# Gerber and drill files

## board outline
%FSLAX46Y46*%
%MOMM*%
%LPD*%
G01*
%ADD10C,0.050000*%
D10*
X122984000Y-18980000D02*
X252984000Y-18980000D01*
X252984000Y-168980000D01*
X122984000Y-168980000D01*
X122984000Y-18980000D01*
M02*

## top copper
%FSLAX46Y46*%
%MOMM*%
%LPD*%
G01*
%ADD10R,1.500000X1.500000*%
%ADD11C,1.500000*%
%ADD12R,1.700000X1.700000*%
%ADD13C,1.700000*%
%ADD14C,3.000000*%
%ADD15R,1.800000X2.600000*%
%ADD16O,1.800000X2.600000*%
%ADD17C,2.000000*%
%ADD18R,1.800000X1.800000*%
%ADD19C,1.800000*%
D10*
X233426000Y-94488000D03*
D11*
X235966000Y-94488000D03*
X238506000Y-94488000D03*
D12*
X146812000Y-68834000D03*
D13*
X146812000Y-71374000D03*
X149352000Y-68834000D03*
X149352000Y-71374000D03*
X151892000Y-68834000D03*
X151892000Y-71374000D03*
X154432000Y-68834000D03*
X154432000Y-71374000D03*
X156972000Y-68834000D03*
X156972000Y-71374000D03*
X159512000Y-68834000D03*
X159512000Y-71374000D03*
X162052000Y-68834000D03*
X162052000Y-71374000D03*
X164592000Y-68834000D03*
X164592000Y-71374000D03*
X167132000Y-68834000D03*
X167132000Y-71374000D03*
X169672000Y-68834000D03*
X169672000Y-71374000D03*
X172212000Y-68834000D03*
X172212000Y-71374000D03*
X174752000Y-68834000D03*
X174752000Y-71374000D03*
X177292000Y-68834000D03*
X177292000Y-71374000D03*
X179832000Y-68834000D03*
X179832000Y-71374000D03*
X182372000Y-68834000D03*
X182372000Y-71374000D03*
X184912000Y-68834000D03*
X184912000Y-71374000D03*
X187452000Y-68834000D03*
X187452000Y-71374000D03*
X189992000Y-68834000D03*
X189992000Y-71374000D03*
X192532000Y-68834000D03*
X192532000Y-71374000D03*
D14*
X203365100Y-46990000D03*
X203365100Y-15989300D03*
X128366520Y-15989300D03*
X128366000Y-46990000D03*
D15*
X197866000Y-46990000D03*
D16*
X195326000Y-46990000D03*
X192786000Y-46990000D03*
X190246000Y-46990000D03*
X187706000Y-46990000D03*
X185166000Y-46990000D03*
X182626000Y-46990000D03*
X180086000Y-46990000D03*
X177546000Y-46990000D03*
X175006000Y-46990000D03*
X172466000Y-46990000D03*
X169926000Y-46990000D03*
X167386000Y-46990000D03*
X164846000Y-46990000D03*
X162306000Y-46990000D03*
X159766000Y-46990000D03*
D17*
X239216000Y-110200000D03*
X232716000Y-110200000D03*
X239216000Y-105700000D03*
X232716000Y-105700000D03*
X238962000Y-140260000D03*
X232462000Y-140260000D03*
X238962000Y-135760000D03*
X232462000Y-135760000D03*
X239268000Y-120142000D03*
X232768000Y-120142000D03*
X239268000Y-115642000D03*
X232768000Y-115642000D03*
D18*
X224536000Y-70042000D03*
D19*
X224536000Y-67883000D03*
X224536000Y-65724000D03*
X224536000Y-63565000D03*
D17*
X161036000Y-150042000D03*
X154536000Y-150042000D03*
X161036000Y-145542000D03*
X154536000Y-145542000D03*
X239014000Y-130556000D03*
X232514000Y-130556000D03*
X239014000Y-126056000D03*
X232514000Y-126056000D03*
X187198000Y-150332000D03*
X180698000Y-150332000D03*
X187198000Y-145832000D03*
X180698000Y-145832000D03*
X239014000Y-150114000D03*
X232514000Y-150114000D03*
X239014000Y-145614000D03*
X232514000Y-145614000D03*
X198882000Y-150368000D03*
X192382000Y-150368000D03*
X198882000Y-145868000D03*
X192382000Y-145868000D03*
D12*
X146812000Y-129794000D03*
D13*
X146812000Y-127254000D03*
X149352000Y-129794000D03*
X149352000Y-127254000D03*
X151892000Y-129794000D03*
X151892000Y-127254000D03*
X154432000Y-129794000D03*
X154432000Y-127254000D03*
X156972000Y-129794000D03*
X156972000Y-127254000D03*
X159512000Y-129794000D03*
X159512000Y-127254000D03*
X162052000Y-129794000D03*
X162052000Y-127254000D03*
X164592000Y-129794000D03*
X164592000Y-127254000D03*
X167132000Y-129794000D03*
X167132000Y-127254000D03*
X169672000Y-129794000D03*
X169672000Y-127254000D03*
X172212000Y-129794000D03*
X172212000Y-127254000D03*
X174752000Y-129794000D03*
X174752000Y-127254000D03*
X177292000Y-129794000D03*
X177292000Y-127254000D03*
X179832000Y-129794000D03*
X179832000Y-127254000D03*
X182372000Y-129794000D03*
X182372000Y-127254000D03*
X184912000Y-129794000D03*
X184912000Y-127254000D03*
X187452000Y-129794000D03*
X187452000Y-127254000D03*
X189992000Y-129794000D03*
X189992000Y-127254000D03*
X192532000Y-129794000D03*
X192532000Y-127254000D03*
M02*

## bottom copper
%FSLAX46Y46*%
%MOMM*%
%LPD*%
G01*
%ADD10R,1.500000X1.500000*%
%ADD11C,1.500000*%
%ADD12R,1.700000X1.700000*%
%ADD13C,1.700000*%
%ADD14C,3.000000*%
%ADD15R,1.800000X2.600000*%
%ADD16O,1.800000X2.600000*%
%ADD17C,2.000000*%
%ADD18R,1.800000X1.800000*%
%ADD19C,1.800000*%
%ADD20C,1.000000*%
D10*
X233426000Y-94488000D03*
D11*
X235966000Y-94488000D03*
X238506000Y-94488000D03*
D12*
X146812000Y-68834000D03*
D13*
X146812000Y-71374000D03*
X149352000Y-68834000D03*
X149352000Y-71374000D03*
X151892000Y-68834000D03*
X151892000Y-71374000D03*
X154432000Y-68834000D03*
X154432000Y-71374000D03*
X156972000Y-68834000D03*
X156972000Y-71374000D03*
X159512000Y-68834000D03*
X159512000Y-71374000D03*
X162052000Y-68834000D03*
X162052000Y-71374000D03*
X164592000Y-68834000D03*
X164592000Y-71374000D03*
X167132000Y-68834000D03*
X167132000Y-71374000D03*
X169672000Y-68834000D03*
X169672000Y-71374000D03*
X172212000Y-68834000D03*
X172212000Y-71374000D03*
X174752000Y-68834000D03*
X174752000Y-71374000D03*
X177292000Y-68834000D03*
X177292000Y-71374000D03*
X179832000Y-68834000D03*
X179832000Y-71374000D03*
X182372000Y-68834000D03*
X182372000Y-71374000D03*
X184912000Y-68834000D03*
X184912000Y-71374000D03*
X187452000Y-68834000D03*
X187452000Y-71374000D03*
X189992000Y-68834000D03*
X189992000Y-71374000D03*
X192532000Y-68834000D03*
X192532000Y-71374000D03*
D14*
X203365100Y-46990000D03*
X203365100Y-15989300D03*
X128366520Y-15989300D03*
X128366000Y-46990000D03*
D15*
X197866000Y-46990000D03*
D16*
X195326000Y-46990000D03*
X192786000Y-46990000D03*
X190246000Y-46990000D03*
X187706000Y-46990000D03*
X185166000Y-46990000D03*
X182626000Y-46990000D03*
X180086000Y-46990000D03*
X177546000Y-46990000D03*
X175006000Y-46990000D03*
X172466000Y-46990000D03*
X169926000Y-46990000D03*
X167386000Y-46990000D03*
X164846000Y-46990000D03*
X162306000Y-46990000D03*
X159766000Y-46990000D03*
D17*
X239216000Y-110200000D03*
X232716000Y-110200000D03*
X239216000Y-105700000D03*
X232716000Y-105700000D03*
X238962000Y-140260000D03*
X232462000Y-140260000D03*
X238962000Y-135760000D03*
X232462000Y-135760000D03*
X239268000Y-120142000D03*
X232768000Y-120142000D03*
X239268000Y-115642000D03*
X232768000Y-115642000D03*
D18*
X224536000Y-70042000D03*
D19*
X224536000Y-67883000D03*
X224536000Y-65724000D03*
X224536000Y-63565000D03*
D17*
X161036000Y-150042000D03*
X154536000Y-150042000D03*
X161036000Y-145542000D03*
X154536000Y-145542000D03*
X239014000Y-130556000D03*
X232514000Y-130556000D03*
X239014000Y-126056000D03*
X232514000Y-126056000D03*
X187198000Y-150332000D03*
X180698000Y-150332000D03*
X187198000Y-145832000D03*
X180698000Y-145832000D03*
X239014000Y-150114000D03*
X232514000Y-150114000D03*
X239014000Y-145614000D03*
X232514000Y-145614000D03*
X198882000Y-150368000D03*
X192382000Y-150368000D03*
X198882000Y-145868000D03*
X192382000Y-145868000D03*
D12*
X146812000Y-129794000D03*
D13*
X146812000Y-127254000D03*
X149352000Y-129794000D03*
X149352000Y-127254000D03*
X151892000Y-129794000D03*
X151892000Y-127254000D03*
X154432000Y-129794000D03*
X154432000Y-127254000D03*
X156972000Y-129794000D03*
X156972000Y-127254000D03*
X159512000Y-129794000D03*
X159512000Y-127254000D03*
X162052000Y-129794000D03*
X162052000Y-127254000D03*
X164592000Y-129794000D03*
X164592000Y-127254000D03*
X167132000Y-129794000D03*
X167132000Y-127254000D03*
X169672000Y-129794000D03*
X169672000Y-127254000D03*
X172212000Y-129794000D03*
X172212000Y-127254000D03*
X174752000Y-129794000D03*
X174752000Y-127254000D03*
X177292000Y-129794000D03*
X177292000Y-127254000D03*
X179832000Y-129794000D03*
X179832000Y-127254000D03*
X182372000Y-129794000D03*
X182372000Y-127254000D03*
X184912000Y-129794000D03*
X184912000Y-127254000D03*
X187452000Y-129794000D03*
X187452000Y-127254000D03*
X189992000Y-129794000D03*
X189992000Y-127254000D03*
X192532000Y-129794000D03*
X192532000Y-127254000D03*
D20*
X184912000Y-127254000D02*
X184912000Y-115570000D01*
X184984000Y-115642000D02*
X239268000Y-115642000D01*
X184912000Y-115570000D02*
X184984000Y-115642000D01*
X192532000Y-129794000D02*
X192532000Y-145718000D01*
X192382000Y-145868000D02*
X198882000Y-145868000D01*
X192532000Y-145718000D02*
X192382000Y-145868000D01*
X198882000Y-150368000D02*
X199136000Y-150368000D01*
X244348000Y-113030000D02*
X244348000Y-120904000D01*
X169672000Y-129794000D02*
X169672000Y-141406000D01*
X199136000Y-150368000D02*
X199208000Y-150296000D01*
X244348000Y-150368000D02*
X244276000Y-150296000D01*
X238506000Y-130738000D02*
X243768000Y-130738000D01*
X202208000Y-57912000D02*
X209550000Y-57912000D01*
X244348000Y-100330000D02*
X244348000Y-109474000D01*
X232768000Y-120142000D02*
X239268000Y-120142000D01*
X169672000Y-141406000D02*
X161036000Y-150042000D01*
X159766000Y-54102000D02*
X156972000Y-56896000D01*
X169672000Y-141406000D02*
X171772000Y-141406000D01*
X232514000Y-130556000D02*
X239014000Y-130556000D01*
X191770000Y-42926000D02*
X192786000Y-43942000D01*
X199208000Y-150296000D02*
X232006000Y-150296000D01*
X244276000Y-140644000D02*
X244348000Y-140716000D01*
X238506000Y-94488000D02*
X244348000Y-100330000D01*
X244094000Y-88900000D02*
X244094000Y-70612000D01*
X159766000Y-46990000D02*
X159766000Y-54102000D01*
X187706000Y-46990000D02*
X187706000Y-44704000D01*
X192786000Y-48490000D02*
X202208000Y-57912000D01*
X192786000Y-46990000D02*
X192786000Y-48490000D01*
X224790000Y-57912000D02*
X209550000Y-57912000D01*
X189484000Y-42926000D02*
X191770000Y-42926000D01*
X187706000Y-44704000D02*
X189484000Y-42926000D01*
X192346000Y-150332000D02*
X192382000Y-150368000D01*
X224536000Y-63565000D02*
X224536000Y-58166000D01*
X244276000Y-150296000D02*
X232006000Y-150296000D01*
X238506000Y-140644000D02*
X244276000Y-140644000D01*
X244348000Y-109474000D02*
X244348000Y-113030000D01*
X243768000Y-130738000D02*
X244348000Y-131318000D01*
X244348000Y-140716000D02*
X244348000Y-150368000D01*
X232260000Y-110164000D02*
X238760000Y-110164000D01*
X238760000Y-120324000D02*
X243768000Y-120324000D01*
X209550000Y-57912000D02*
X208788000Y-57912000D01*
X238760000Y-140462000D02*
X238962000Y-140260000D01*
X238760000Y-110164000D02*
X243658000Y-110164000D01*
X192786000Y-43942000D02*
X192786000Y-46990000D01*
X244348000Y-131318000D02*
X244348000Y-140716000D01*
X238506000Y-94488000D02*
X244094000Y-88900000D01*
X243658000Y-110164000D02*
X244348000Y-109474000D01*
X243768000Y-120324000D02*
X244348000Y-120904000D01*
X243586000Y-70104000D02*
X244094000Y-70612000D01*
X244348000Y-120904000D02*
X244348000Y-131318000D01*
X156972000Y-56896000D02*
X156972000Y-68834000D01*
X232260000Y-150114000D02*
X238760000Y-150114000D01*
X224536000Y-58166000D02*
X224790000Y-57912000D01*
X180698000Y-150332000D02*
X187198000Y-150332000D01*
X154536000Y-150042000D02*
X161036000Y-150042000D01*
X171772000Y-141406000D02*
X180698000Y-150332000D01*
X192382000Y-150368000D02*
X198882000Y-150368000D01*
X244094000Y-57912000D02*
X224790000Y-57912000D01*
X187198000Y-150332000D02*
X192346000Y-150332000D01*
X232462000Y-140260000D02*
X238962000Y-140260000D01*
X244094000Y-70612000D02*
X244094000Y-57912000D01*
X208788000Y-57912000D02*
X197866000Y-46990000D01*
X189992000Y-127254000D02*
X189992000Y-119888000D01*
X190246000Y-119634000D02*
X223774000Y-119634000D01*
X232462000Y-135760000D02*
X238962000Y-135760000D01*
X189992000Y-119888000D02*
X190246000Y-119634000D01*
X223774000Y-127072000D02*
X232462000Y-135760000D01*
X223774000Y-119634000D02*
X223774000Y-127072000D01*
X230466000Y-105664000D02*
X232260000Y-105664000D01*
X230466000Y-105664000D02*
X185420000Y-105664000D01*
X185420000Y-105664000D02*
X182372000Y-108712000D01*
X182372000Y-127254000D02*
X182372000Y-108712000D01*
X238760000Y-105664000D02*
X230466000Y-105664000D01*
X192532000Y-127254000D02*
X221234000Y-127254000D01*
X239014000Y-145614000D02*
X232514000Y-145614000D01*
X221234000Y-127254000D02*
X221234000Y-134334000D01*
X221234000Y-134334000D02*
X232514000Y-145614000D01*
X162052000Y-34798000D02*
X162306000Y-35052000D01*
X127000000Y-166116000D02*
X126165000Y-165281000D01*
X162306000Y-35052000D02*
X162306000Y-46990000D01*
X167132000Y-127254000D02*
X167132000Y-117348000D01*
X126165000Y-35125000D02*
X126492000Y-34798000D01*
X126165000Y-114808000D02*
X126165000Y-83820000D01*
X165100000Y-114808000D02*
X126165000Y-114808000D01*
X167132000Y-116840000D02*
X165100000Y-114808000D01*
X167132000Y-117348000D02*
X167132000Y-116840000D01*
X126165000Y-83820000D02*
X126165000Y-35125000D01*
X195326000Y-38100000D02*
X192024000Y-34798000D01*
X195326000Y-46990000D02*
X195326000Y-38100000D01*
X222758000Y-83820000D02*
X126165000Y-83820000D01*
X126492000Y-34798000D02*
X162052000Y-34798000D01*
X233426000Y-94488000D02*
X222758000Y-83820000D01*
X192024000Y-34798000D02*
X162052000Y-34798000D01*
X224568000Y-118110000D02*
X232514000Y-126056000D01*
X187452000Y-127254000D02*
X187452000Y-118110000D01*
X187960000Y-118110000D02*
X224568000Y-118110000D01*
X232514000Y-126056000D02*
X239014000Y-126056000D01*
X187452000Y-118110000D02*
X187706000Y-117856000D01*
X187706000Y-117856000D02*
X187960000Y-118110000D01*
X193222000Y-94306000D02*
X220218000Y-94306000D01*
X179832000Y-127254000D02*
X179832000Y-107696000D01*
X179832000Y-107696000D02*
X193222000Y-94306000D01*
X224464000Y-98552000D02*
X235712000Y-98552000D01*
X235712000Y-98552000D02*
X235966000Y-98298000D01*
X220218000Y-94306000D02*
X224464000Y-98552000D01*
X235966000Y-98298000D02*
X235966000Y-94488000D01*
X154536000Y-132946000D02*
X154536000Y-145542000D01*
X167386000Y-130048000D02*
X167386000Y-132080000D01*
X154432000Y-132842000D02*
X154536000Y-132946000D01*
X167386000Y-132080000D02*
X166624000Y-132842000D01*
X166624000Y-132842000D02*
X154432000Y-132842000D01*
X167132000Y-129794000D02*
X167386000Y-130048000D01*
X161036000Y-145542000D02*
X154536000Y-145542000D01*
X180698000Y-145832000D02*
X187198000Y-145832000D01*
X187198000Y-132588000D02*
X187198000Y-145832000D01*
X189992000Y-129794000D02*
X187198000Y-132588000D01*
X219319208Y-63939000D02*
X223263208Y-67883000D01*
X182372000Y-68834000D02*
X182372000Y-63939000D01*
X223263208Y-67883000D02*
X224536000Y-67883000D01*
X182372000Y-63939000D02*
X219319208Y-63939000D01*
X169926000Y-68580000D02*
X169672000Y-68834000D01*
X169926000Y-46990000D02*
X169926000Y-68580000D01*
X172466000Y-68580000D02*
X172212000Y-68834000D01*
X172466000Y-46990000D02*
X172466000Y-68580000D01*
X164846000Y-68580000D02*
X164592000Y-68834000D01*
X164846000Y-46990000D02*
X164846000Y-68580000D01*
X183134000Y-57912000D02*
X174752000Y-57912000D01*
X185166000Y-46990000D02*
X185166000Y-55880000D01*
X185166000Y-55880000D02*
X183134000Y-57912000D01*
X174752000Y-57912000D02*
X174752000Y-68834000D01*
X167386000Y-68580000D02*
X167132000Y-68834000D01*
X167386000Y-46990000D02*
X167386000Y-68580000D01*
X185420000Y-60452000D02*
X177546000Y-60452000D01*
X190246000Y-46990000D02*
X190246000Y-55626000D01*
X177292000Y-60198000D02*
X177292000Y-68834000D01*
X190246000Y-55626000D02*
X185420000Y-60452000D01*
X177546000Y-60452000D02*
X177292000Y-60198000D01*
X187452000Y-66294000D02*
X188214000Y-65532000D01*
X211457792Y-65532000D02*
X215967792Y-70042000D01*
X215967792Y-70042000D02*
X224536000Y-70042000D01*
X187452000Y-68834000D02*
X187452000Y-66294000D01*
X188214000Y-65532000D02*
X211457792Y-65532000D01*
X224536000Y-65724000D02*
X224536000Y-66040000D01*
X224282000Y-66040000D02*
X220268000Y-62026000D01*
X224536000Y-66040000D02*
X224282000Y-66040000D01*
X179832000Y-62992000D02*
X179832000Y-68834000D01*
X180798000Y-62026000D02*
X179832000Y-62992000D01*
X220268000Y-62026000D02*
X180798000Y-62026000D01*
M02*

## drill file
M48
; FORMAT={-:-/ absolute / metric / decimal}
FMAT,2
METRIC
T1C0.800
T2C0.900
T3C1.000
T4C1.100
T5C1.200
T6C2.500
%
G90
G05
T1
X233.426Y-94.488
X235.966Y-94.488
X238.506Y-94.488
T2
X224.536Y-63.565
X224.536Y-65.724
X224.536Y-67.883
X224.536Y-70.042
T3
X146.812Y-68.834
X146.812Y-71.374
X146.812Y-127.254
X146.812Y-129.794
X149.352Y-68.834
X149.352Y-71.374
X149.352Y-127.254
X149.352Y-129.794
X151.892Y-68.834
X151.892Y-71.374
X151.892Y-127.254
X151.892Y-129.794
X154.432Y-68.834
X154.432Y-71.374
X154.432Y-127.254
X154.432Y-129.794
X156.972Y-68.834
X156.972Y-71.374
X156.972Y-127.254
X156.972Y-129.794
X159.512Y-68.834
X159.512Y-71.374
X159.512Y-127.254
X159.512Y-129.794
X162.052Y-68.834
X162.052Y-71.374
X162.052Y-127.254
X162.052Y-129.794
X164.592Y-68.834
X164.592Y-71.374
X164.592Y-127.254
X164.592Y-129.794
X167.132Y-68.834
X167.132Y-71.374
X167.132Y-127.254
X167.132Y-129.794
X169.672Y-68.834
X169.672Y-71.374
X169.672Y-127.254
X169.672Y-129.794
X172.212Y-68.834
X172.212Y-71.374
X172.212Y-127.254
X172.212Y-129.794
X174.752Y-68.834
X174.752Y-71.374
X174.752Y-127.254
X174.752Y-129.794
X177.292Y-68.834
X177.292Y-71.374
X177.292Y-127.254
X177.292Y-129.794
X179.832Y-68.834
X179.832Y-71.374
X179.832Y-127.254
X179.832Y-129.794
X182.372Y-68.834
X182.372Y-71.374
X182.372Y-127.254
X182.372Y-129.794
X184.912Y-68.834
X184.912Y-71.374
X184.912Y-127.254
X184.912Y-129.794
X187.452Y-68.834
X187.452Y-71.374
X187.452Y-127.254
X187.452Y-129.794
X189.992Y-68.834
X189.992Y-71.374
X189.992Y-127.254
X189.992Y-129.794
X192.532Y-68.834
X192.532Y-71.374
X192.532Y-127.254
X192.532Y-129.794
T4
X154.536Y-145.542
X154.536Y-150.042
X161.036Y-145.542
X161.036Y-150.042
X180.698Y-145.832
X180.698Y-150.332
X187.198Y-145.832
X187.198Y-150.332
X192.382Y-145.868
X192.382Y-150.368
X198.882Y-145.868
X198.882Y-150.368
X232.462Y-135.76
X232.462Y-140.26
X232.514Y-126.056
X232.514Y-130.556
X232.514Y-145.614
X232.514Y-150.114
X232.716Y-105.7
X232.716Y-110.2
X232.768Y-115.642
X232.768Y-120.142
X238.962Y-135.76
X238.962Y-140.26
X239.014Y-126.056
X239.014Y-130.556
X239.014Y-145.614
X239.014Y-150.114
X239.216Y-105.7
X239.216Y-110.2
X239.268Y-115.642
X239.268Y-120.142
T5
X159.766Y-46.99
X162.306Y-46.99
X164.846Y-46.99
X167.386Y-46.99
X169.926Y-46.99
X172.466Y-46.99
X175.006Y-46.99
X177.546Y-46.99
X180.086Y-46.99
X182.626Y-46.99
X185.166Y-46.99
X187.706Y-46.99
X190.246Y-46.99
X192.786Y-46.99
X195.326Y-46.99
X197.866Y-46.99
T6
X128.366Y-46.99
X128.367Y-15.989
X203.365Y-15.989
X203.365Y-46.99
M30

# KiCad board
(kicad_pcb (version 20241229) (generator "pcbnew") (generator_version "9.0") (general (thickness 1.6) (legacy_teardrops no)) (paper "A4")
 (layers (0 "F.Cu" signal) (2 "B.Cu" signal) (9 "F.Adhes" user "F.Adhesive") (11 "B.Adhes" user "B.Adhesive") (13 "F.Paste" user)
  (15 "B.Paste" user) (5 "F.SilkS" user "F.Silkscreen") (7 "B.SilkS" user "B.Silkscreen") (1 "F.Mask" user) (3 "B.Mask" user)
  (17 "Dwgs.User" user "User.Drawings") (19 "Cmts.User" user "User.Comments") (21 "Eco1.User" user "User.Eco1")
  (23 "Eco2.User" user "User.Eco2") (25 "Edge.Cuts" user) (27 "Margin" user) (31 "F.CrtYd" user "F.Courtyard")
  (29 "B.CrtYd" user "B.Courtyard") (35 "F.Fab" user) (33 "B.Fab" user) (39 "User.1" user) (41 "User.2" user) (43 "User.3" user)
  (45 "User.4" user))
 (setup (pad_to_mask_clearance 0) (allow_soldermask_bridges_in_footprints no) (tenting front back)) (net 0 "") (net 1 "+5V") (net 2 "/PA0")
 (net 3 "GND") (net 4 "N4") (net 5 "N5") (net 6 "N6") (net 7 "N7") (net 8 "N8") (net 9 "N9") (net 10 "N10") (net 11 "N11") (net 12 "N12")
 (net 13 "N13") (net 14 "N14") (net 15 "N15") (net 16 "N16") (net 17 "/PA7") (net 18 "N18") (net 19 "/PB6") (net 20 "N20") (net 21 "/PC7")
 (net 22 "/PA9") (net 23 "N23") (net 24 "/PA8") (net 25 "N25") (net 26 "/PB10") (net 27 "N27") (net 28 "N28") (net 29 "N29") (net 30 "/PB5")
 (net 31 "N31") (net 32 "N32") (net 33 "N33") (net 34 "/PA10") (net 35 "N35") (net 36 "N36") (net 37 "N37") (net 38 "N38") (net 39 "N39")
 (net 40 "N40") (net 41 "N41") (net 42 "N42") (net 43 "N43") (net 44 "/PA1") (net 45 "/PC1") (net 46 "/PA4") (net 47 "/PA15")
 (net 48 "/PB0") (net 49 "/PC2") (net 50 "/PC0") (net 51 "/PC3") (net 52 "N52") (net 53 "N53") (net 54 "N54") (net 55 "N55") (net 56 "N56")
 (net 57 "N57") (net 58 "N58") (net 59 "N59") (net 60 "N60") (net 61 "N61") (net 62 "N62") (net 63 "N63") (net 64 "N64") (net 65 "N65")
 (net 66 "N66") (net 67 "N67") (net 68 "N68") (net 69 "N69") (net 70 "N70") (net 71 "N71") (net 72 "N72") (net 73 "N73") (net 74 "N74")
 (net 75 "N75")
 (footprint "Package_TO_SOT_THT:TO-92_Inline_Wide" (layer "F.Cu") (at 233.426 94.488)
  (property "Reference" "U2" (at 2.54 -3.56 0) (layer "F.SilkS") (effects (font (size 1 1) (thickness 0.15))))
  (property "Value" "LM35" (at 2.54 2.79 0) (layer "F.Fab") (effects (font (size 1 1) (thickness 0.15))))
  (pad "1" thru_hole rect (at 0 0) (size 1.5 1.5) (drill 0.8) (layers "*.Cu" "*.Mask") (remove_unused_layers no) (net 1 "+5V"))
  (pad "2" thru_hole circle (at 2.54 0) (size 1.5 1.5) (drill 0.8) (layers "*.Cu" "*.Mask") (remove_unused_layers no) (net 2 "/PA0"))
  (pad "3" thru_hole circle (at 5.08 0) (size 1.5 1.5) (drill 0.8) (layers "*.Cu" "*.Mask") (remove_unused_layers no) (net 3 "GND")))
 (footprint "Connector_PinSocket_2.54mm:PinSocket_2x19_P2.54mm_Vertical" (layer "F.Cu") (at 146.812 68.834 90)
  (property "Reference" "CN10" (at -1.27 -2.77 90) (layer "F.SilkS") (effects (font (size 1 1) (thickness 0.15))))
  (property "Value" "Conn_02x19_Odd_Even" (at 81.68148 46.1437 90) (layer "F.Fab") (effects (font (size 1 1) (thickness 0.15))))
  (pad "1" thru_hole rect (at 0 0 90) (size 1.7 1.7) (drill 1) (layers "*.Cu" "*.Mask") (remove_unused_layers no) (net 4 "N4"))
  (pad "2" thru_hole circle (at -2.54 0 90) (size 1.7 1.7) (drill 1) (layers "*.Cu" "*.Mask") (remove_unused_layers no) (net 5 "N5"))
  (pad "3" thru_hole circle (at 0 2.54 90) (size 1.7 1.7) (drill 1) (layers "*.Cu" "*.Mask") (remove_unused_layers no) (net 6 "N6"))
  (pad "4" thru_hole circle (at -2.54 2.54 90) (size 1.7 1.7) (drill 1) (layers "*.Cu" "*.Mask") (remove_unused_layers no) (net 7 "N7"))
  (pad "5" thru_hole circle (at 0 5.08 90) (size 1.7 1.7) (drill 1) (layers "*.Cu" "*.Mask") (remove_unused_layers no) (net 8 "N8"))
  (pad "6" thru_hole circle (at -2.54 5.08 90) (size 1.7 1.7) (drill 1) (layers "*.Cu" "*.Mask") (remove_unused_layers no) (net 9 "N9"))
  (pad "7" thru_hole circle (at 0 7.62 90) (size 1.7 1.7) (drill 1) (layers "*.Cu" "*.Mask") (remove_unused_layers no) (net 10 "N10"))
  (pad "8" thru_hole circle (at -2.54 7.62 90) (size 1.7 1.7) (drill 1) (layers "*.Cu" "*.Mask") (remove_unused_layers no) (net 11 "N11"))
  (pad "9" thru_hole circle (at 0 10.16 90) (size 1.7 1.7) (drill 1) (layers "*.Cu" "*.Mask") (remove_unused_layers no) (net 3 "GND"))
  (pad "10" thru_hole circle (at -2.54 10.16 90) (size 1.7 1.7) (drill 1) (layers "*.Cu" "*.Mask") (remove_unused_layers no) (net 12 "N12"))
  (pad "11" thru_hole circle (at 0 12.7 90) (size 1.7 1.7) (drill 1) (layers "*.Cu" "*.Mask") (remove_unused_layers no) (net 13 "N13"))
  (pad "12" thru_hole circle (at -2.54 12.7 90) (size 1.7 1.7) (drill 1) (layers "*.Cu" "*.Mask") (remove_unused_layers no) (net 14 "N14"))
  (pad "13" thru_hole circle (at 0 15.24 90) (size 1.7 1.7) (drill 1) (layers "*.Cu" "*.Mask") (remove_unused_layers no) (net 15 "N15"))
  (pad "14" thru_hole circle (at -2.54 15.24 90) (size 1.7 1.7) (drill 1) (layers "*.Cu" "*.Mask") (remove_unused_layers no) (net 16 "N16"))
  (pad "15" thru_hole circle (at 0 17.78 90) (size 1.7 1.7) (drill 1) (layers "*.Cu" "*.Mask") (remove_unused_layers no) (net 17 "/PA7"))
  (pad "16" thru_hole circle (at -2.54 17.78 90) (size 1.7 1.7) (drill 1) (layers "*.Cu" "*.Mask") (remove_unused_layers no) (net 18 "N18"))
  (pad "17" thru_hole circle (at 0 20.32 90) (size 1.7 1.7) (drill 1) (layers "*.Cu" "*.Mask") (remove_unused_layers no) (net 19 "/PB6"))
  (pad "18" thru_hole circle (at -2.54 20.32 90) (size 1.7 1.7) (drill 1) (layers "*.Cu" "*.Mask") (remove_unused_layers no) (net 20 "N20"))
  (pad "19" thru_hole circle (at 0 22.86 90) (size 1.7 1.7) (drill 1) (layers "*.Cu" "*.Mask") (remove_unused_layers no) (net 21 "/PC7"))
  (pad "20" thru_hole circle (at -2.54 22.86 90) (size 1.7 1.7) (drill 1) (layers "*.Cu" "*.Mask") (remove_unused_layers no) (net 3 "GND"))
  (pad "21" thru_hole circle (at 0 25.4 90) (size 1.7 1.7) (drill 1) (layers "*.Cu" "*.Mask") (remove_unused_layers no) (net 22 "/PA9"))
  (pad "22" thru_hole circle (at -2.54 25.4 90) (size 1.7 1.7) (drill 1) (layers "*.Cu" "*.Mask") (remove_unused_layers no) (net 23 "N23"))
  (pad "23" thru_hole circle (at 0 27.94 90) (size 1.7 1.7) (drill 1) (layers "*.Cu" "*.Mask") (remove_unused_layers no) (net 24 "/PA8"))
  (pad "24" thru_hole circle (at -2.54 27.94 90) (size 1.7 1.7) (drill 1) (layers "*.Cu" "*.Mask") (remove_unused_layers no) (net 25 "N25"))
  (pad "25" thru_hole circle (at 0 30.48 90) (size 1.7 1.7) (drill 1) (layers "*.Cu" "*.Mask") (remove_unused_layers no) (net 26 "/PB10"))
  (pad "26" thru_hole circle (at -2.54 30.48 90) (size 1.7 1.7) (drill 1) (layers "*.Cu" "*.Mask") (remove_unused_layers no) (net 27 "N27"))
  (pad "27" thru_hole circle (at 0 33.02 90) (size 1.7 1.7) (drill 1) (layers "*.Cu" "*.Mask") (remove_unused_layers no) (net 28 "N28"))
  (pad "28" thru_hole circle (at -2.54 33.02 90) (size 1.7 1.7) (drill 1) (layers "*.Cu" "*.Mask") (remove_unused_layers no) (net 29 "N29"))
  (pad "29" thru_hole circle (at 0 35.56 90) (size 1.7 1.7) (drill 1) (layers "*.Cu" "*.Mask") (remove_unused_layers no) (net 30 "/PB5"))
  (pad "30" thru_hole circle (at -2.54 35.56 90) (size 1.7 1.7) (drill 1) (layers "*.Cu" "*.Mask") (remove_unused_layers no) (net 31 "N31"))
  (pad "31" thru_hole circle (at 0 38.1 90) (size 1.7 1.7) (drill 1) (layers "*.Cu" "*.Mask") (remove_unused_layers no) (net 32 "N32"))
  (pad "32" thru_hole circle (at -2.54 38.1 90) (size 1.7 1.7) (drill 1) (layers "*.Cu" "*.Mask") (remove_unused_layers no) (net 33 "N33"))
  (pad "33" thru_hole circle (at 0 40.64 90) (size 1.7 1.7) (drill 1) (layers "*.Cu" "*.Mask") (remove_unused_layers no) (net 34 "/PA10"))
  (pad "34" thru_hole circle (at -2.54 40.64 90) (size 1.7 1.7) (drill 1) (layers "*.Cu" "*.Mask") (remove_unused_layers no) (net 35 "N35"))
  (pad "35" thru_hole circle (at 0 43.18 90) (size 1.7 1.7) (drill 1) (layers "*.Cu" "*.Mask") (remove_unused_layers no) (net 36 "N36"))
  (pad "36" thru_hole circle (at -2.54 43.18 90) (size 1.7 1.7) (drill 1) (layers "*.Cu" "*.Mask") (remove_unused_layers no) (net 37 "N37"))
  (pad "37" thru_hole circle (at 0 45.72 90) (size 1.7 1.7) (drill 1) (layers "*.Cu" "*.Mask") (remove_unused_layers no) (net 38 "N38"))
  (pad "38" thru_hole circle (at -2.54 45.72 90) (size 1.7 1.7) (drill 1) (layers "*.Cu" "*.Mask") (remove_unused_layers no) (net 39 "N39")))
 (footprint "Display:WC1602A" (layer "F.Cu") (at 197.866 46.99 180)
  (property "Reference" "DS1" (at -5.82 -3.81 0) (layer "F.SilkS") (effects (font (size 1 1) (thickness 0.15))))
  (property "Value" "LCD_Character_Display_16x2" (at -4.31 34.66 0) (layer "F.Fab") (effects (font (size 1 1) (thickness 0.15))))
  (pad "" thru_hole circle (at -5.4991 0 180) (size 3 3) (drill 2.5) (layers "*.Cu" "*.Mask") (remove_unused_layers no))
  (pad "" thru_hole circle (at -5.4991 31.0007 180) (size 3 3) (drill 2.5) (layers "*.Cu" "*.Mask") (remove_unused_layers no))
  (pad "" thru_hole circle (at 69.49948 31.0007 180) (size 3 3) (drill 2.5) (layers "*.Cu" "*.Mask") (remove_unused_layers no))
  (pad "" thru_hole circle (at 69.5 0 180) (size 3 3) (drill 2.5) (layers "*.Cu" "*.Mask") (remove_unused_layers no))
  (pad "1" thru_hole rect (at 0 0 180) (size 1.8 2.6) (drill 1.2) (layers "*.Cu" "*.Mask") (remove_unused_layers no) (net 3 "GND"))
  (pad "2" thru_hole oval (at 2.54 0 180) (size 1.8 2.6) (drill 1.2) (layers "*.Cu" "*.Mask") (remove_unused_layers no) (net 1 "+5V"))
  (pad "3" thru_hole oval (at 5.08 0 180) (size 1.8 2.6) (drill 1.2) (layers "*.Cu" "*.Mask") (remove_unused_layers no) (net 3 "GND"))
  (pad "4" thru_hole oval (at 7.62 0 180) (size 1.8 2.6) (drill 1.2) (layers "*.Cu" "*.Mask") (remove_unused_layers no) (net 26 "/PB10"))
  (pad "5" thru_hole oval (at 10.16 0 180) (size 1.8 2.6) (drill 1.2) (layers "*.Cu" "*.Mask") (remove_unused_layers no) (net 3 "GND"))
  (pad "6" thru_hole oval (at 12.7 0 180) (size 1.8 2.6) (drill 1.2) (layers "*.Cu" "*.Mask") (remove_unused_layers no) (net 24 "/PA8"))
  (pad "7" thru_hole oval (at 15.24 0 180) (size 1.8 2.6) (drill 1.2) (layers "*.Cu" "*.Mask") (remove_unused_layers no) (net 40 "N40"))
  (pad "8" thru_hole oval (at 17.78 0 180) (size 1.8 2.6) (drill 1.2) (layers "*.Cu" "*.Mask") (remove_unused_layers no) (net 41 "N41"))
  (pad "9" thru_hole oval (at 20.32 0 180) (size 1.8 2.6) (drill 1.2) (layers "*.Cu" "*.Mask") (remove_unused_layers no) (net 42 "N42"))
  (pad "10" thru_hole oval (at 22.86 0 180) (size 1.8 2.6) (drill 1.2) (layers "*.Cu" "*.Mask") (remove_unused_layers no) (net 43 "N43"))
  (pad "11" thru_hole oval (at 25.4 0 180) (size 1.8 2.6) (drill 1.2) (layers "*.Cu" "*.Mask") (remove_unused_layers no) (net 22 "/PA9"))
  (pad "12" thru_hole oval (at 27.94 0 180) (size 1.8 2.6) (drill 1.2) (layers "*.Cu" "*.Mask") (remove_unused_layers no) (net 21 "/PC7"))
  (pad "13" thru_hole oval (at 30.48 0 180) (size 1.8 2.6) (drill 1.2) (layers "*.Cu" "*.Mask") (remove_unused_layers no) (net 19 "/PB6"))
  (pad "14" thru_hole oval (at 33.02 0 180) (size 1.8 2.6) (drill 1.2) (layers "*.Cu" "*.Mask") (remove_unused_layers no) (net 17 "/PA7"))
  (pad "15" thru_hole oval (at 35.56 0 180) (size 1.8 2.6) (drill 1.2) (layers "*.Cu" "*.Mask") (remove_unused_layers no) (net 1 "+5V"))
  (pad "16" thru_hole oval (at 38.1 0 180) (size 1.8 2.6) (drill 1.2) (layers "*.Cu" "*.Mask") (remove_unused_layers no) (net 3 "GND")))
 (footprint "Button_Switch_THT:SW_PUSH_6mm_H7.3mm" (layer "F.Cu") (at 239.216 110.2 180)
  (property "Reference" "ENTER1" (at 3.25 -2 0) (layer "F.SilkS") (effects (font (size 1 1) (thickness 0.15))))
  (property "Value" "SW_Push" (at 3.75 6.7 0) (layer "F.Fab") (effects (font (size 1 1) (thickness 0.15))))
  (pad "1" thru_hole circle (at 0 0 270) (size 2 2) (drill 1.1) (layers "*.Cu" "*.Mask") (remove_unused_layers no) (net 3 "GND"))
  (pad "1" thru_hole circle (at 6.5 0 270) (size 2 2) (drill 1.1) (layers "*.Cu" "*.Mask") (remove_unused_layers no) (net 3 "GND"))
  (pad "2" thru_hole circle (at 0 4.5 270) (size 2 2) (drill 1.1) (layers "*.Cu" "*.Mask") (remove_unused_layers no) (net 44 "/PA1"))
  (pad "2" thru_hole circle (at 6.5 4.5 270) (size 2 2) (drill 1.1) (layers "*.Cu" "*.Mask") (remove_unused_layers no) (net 44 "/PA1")))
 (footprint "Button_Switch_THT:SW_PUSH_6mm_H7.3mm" (layer "F.Cu") (at 238.962 140.26 180)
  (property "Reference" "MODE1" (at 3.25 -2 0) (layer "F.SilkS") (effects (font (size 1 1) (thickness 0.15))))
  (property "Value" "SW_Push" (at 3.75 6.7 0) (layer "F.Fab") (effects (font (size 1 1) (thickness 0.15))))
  (pad "1" thru_hole circle (at 0 0 270) (size 2 2) (drill 1.1) (layers "*.Cu" "*.Mask") (remove_unused_layers no) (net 3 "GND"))
  (pad "1" thru_hole circle (at 6.5 0 270) (size 2 2) (drill 1.1) (layers "*.Cu" "*.Mask") (remove_unused_layers no) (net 3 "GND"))
  (pad "2" thru_hole circle (at 0 4.5 270) (size 2 2) (drill 1.1) (layers "*.Cu" "*.Mask") (remove_unused_layers no) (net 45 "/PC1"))
  (pad "2" thru_hole circle (at 6.5 4.5 270) (size 2 2) (drill 1.1) (layers "*.Cu" "*.Mask") (remove_unused_layers no) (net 45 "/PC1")))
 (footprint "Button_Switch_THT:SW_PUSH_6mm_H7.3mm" (layer "F.Cu") (at 239.268 120.142 180)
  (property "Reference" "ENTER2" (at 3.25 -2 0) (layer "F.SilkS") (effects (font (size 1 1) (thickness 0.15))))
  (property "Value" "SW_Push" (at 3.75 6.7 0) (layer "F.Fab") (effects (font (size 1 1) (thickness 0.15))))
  (pad "1" thru_hole circle (at 0 0 270) (size 2 2) (drill 1.1) (layers "*.Cu" "*.Mask") (remove_unused_layers no) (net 3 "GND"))
  (pad "1" thru_hole circle (at 6.5 0 270) (size 2 2) (drill 1.1) (layers "*.Cu" "*.Mask") (remove_unused_layers no) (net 3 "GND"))
  (pad "2" thru_hole circle (at 0 4.5 270) (size 2 2) (drill 1.1) (layers "*.Cu" "*.Mask") (remove_unused_layers no) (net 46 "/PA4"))
  (pad "2" thru_hole circle (at 6.5 4.5 270) (size 2 2) (drill 1.1) (layers "*.Cu" "*.Mask") (remove_unused_layers no) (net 46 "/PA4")))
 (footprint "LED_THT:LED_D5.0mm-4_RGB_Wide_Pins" (layer "F.Cu") (at 224.536 70.042 90)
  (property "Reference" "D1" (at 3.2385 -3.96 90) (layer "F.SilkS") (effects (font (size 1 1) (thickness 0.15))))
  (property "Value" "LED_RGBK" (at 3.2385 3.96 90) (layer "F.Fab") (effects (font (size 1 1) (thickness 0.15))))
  (pad "1" thru_hole rect (at 0 0 90) (size 1.8 1.8) (drill 0.9) (layers "*.Cu" "*.Mask") (remove_unused_layers no) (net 34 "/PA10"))
  (pad "2" thru_hole circle (at 2.159 0 90) (size 1.8 1.8) (drill 0.9) (layers "*.Cu" "*.Mask") (remove_unused_layers no) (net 30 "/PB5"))
  (pad "3" thru_hole circle (at 4.318 0 90) (size 1.8 1.8) (drill 0.9) (layers "*.Cu" "*.Mask") (remove_unused_layers no) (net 28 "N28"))
  (pad "4" thru_hole circle (at 6.477 0 90) (size 1.8 1.8) (drill 0.9) (layers "*.Cu" "*.Mask") (remove_unused_layers no) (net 3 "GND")))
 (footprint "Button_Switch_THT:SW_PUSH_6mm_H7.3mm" (layer "F.Cu") (at 161.036 150.042 180)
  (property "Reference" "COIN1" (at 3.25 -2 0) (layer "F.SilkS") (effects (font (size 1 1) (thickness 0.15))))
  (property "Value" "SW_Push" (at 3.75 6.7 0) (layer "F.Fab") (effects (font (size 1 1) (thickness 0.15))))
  (pad "1" thru_hole circle (at 0 0 270) (size 2 2) (drill 1.1) (layers "*.Cu" "*.Mask") (remove_unused_layers no) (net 3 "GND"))
  (pad "1" thru_hole circle (at 6.5 0 270) (size 2 2) (drill 1.1) (layers "*.Cu" "*.Mask") (remove_unused_layers no) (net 3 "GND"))
  (pad "2" thru_hole circle (at 0 4.5 270) (size 2 2) (drill 1.1) (layers "*.Cu" "*.Mask") (remove_unused_layers no) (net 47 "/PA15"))
  (pad "2" thru_hole circle (at 6.5 4.5 270) (size 2 2) (drill 1.1) (layers "*.Cu" "*.Mask") (remove_unused_layers no) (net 47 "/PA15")))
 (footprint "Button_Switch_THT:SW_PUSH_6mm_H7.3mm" (layer "F.Cu") (at 239.014 130.556 180)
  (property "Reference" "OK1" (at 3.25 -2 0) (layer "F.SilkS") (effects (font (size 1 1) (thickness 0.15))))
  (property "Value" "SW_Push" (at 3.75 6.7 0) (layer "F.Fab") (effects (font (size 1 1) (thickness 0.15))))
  (pad "1" thru_hole circle (at 0 0 270) (size 2 2) (drill 1.1) (layers "*.Cu" "*.Mask") (remove_unused_layers no) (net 3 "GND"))
  (pad "1" thru_hole circle (at 6.5 0 270) (size 2 2) (drill 1.1) (layers "*.Cu" "*.Mask") (remove_unused_layers no) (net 3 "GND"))
  (pad "2" thru_hole circle (at 0 4.5 270) (size 2 2) (drill 1.1) (layers "*.Cu" "*.Mask") (remove_unused_layers no) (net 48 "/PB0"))
  (pad "2" thru_hole circle (at 6.5 4.5 270) (size 2 2) (drill 1.1) (layers "*.Cu" "*.Mask") (remove_unused_layers no) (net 48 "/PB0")))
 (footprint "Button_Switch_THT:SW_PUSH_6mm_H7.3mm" (layer "F.Cu") (at 187.198 150.332 180)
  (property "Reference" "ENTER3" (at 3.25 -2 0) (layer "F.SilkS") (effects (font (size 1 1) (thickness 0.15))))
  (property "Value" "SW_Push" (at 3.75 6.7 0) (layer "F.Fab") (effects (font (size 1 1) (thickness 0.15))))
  (pad "1" thru_hole circle (at 0 0 270) (size 2 2) (drill 1.1) (layers "*.Cu" "*.Mask") (remove_unused_layers no) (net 3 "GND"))
  (pad "1" thru_hole circle (at 6.5 0 270) (size 2 2) (drill 1.1) (layers "*.Cu" "*.Mask") (remove_unused_layers no) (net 3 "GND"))
  (pad "2" thru_hole circle (at 0 4.5 270) (size 2 2) (drill 1.1) (layers "*.Cu" "*.Mask") (remove_unused_layers no) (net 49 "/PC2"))
  (pad "2" thru_hole circle (at 6.5 4.5 270) (size 2 2) (drill 1.1) (layers "*.Cu" "*.Mask") (remove_unused_layers no) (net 49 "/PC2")))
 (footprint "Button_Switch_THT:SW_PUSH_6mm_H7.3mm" (layer "F.Cu") (at 239.014 150.114 180)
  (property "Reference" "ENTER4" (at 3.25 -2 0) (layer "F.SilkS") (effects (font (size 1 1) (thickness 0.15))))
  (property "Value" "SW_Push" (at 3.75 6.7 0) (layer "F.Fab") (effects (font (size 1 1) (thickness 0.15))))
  (pad "1" thru_hole circle (at 0 0 270) (size 2 2) (drill 1.1) (layers "*.Cu" "*.Mask") (remove_unused_layers no) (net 3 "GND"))
  (pad "1" thru_hole circle (at 6.5 0 270) (size 2 2) (drill 1.1) (layers "*.Cu" "*.Mask") (remove_unused_layers no) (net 3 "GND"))
  (pad "2" thru_hole circle (at 0 4.5 270) (size 2 2) (drill 1.1) (layers "*.Cu" "*.Mask") (remove_unused_layers no) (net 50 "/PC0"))
  (pad "2" thru_hole circle (at 6.5 4.5 270) (size 2 2) (drill 1.1) (layers "*.Cu" "*.Mask") (remove_unused_layers no) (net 50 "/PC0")))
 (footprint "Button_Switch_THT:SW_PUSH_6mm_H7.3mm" (layer "F.Cu") (at 198.882 150.368 180)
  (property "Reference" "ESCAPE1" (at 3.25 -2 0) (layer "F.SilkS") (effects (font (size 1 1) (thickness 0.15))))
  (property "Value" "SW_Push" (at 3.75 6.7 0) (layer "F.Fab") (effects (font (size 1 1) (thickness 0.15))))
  (pad "1" thru_hole circle (at 0 0 270) (size 2 2) (drill 1.1) (layers "*.Cu" "*.Mask") (remove_unused_layers no) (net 3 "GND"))
  (pad "1" thru_hole circle (at 6.5 0 270) (size 2 2) (drill 1.1) (layers "*.Cu" "*.Mask") (remove_unused_layers no) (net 3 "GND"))
  (pad "2" thru_hole circle (at 0 4.5 270) (size 2 2) (drill 1.1) (layers "*.Cu" "*.Mask") (remove_unused_layers no) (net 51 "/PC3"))
  (pad "2" thru_hole circle (at 6.5 4.5 270) (size 2 2) (drill 1.1) (layers "*.Cu" "*.Mask") (remove_unused_layers no) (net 51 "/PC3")))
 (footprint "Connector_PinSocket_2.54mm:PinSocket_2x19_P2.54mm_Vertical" (layer "B.Cu") (at 146.812 129.794 -90)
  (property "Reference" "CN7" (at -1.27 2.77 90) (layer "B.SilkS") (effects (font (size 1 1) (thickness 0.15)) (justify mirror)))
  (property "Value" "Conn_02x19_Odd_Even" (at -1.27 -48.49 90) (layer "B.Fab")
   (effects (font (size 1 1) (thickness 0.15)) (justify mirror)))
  (pad "1" thru_hole rect (at 0 0 270) (size 1.7 1.7) (drill 1) (layers "*.Cu" "*.Mask") (remove_unused_layers no) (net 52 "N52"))
  (pad "2" thru_hole circle (at -2.54 0 270) (size 1.7 1.7) (drill 1) (layers "*.Cu" "*.Mask") (remove_unused_layers no) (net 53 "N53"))
  (pad "3" thru_hole circle (at 0 -2.54 270) (size 1.7 1.7) (drill 1) (layers "*.Cu" "*.Mask") (remove_unused_layers no) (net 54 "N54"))
  (pad "4" thru_hole circle (at -2.54 -2.54 270) (size 1.7 1.7) (drill 1) (layers "*.Cu" "*.Mask") (remove_unused_layers no) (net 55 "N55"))
  (pad "5" thru_hole circle (at 0 -5.08 270) (size 1.7 1.7) (drill 1) (layers "*.Cu" "*.Mask") (remove_unused_layers no) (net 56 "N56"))
  (pad "6" thru_hole circle (at -2.54 -5.08 270) (size 1.7 1.7) (drill 1) (layers "*.Cu" "*.Mask") (remove_unused_layers no) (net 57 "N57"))
  (pad "7" thru_hole circle (at 0 -7.62 270) (size 1.7 1.7) (drill 1) (layers "*.Cu" "*.Mask") (remove_unused_layers no) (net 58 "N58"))
  (pad "8" thru_hole circle (at -2.54 -7.62 270) (size 1.7 1.7) (drill 1) (layers "*.Cu" "*.Mask") (remove_unused_layers no) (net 3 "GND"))
  (pad "9" thru_hole circle (at 0 -10.16 270) (size 1.7 1.7) (drill 1) (layers "*.Cu" "*.Mask") (remove_unused_layers no) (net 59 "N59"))
  (pad "10" thru_hole circle (at -2.54 -10.16 270) (size 1.7 1.7) (drill 1) (layers "*.Cu" "*.Mask") (remove_unused_layers no)
   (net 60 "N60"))
  (pad "11" thru_hole circle (at 0 -12.7 270) (size 1.7 1.7) (drill 1) (layers "*.Cu" "*.Mask") (remove_unused_layers no) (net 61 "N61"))
  (pad "12" thru_hole circle (at -2.54 -12.7 270) (size 1.7 1.7) (drill 1) (layers "*.Cu" "*.Mask") (remove_unused_layers no) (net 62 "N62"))
  (pad "13" thru_hole circle (at 0 -15.24 270) (size 1.7 1.7) (drill 1) (layers "*.Cu" "*.Mask") (remove_unused_layers no) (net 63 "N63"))
  (pad "14" thru_hole circle (at -2.54 -15.24 270) (size 1.7 1.7) (drill 1) (layers "*.Cu" "*.Mask") (remove_unused_layers no)
   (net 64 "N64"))
  (pad "15" thru_hole circle (at 0 -17.78 270) (size 1.7 1.7) (drill 1) (layers "*.Cu" "*.Mask") (remove_unused_layers no) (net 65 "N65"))
  (pad "16" thru_hole circle (at -2.54 -17.78 270) (size 1.7 1.7) (drill 1) (layers "*.Cu" "*.Mask") (remove_unused_layers no)
   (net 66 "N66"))
  (pad "17" thru_hole circle (at 0 -20.32 270) (size 1.7 1.7) (drill 1) (layers "*.Cu" "*.Mask") (remove_unused_layers no) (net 47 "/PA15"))
  (pad "18" thru_hole circle (at -2.54 -20.32 270) (size 1.7 1.7) (drill 1) (layers "*.Cu" "*.Mask") (remove_unused_layers no) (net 1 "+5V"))
  (pad "19" thru_hole circle (at 0 -22.86 270) (size 1.7 1.7) (drill 1) (layers "*.Cu" "*.Mask") (remove_unused_layers no) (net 3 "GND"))
  (pad "20" thru_hole circle (at -2.54 -22.86 270) (size 1.7 1.7) (drill 1) (layers "*.Cu" "*.Mask") (remove_unused_layers no) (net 3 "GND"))
  (pad "21" thru_hole circle (at 0 -25.4 270) (size 1.7 1.7) (drill 1) (layers "*.Cu" "*.Mask") (remove_unused_layers no) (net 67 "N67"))
  (pad "22" thru_hole circle (at -2.54 -25.4 270) (size 1.7 1.7) (drill 1) (layers "*.Cu" "*.Mask") (remove_unused_layers no) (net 3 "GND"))
  (pad "23" thru_hole circle (at 0 -27.94 270) (size 1.7 1.7) (drill 1) (layers "*.Cu" "*.Mask") (remove_unused_layers no) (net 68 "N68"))
  (pad "24" thru_hole circle (at -2.54 -27.94 270) (size 1.7 1.7) (drill 1) (layers "*.Cu" "*.Mask") (remove_unused_layers no)
   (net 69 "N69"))
  (pad "25" thru_hole circle (at 0 -30.48 270) (size 1.7 1.7) (drill 1) (layers "*.Cu" "*.Mask") (remove_unused_layers no) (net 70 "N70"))
  (pad "26" thru_hole circle (at -2.54 -30.48 270) (size 1.7 1.7) (drill 1) (layers "*.Cu" "*.Mask") (remove_unused_layers no)
   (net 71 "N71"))
  (pad "27" thru_hole circle (at 0 -33.02 270) (size 1.7 1.7) (drill 1) (layers "*.Cu" "*.Mask") (remove_unused_layers no) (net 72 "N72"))
  (pad "28" thru_hole circle (at -2.54 -33.02 270) (size 1.7 1.7) (drill 1) (layers "*.Cu" "*.Mask") (remove_unused_layers no)
   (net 2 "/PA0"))
  (pad "29" thru_hole circle (at 0 -35.56 270) (size 1.7 1.7) (drill 1) (layers "*.Cu" "*.Mask") (remove_unused_layers no) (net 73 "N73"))
  (pad "30" thru_hole circle (at -2.54 -35.56 270) (size 1.7 1.7) (drill 1) (layers "*.Cu" "*.Mask") (remove_unused_layers no)
   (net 44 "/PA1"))
  (pad "31" thru_hole circle (at 0 -38.1 270) (size 1.7 1.7) (drill 1) (layers "*.Cu" "*.Mask") (remove_unused_layers no) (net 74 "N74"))
  (pad "32" thru_hole circle (at -2.54 -38.1 270) (size 1.7 1.7) (drill 1) (layers "*.Cu" "*.Mask") (remove_unused_layers no)
   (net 46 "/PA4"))
  (pad "33" thru_hole circle (at 0 -40.64 270) (size 1.7 1.7) (drill 1) (layers "*.Cu" "*.Mask") (remove_unused_layers no) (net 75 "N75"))
  (pad "34" thru_hole circle (at -2.54 -40.64 270) (size 1.7 1.7) (drill 1) (layers "*.Cu" "*.Mask") (remove_unused_layers no)
   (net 48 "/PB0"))
  (pad "35" thru_hole circle (at 0 -43.18 270) (size 1.7 1.7) (drill 1) (layers "*.Cu" "*.Mask") (remove_unused_layers no) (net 49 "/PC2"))
  (pad "36" thru_hole circle (at -2.54 -43.18 270) (size 1.7 1.7) (drill 1) (layers "*.Cu" "*.Mask") (remove_unused_layers no)
   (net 45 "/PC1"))
  (pad "37" thru_hole circle (at 0 -45.72 270) (size 1.7 1.7) (drill 1) (layers "*.Cu" "*.Mask") (remove_unused_layers no) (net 51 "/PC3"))
  (pad "38" thru_hole circle (at -2.54 -45.72 270) (size 1.7 1.7) (drill 1) (layers "*.Cu" "*.Mask") (remove_unused_layers no)
   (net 50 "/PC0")))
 (gr_rect (start 122.984 18.98) (end 252.984 168.98) (stroke (width 0.05) (type default)) (fill no) (layer "Edge.Cuts"))
 (segment (start 184.912 127.254) (end 184.912 115.57) (width 1) (layer "B.Cu") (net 46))
 (segment (start 184.984 115.642) (end 239.268 115.642) (width 1) (layer "B.Cu") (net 46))
 (segment (start 184.912 115.57) (end 184.984 115.642) (width 1) (layer "B.Cu") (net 46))
 (segment (start 192.532 129.794) (end 192.532 145.718) (width 1) (layer "B.Cu") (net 51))
 (segment (start 192.382 145.868) (end 198.882 145.868) (width 1) (layer "B.Cu") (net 51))
 (segment (start 192.532 145.718) (end 192.382 145.868) (width 1) (layer "B.Cu") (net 51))
 (segment (start 198.882 150.368) (end 199.136 150.368) (width 1) (layer "B.Cu") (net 3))
 (segment (start 244.348 113.03) (end 244.348 120.904) (width 1) (layer "B.Cu") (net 3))
 (segment (start 169.672 129.794) (end 169.672 141.406) (width 1) (layer "B.Cu") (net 3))
 (segment (start 199.136 150.368) (end 199.208 150.296) (width 1) (layer "B.Cu") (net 3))
 (segment (start 244.348 150.368) (end 244.276 150.296) (width 1) (layer "B.Cu") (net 3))
 (segment (start 238.506 130.738) (end 243.768 130.738) (width 1) (layer "B.Cu") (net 3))
 (segment (start 202.208 57.912) (end 209.55 57.912) (width 1) (layer "B.Cu") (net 3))
 (segment (start 244.348 100.33) (end 244.348 109.474) (width 1) (layer "B.Cu") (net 3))
 (segment (start 232.768 120.142) (end 239.268 120.142) (width 1) (layer "B.Cu") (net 3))
 (segment (start 169.672 141.406) (end 161.036 150.042) (width 1) (layer "B.Cu") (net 3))
 (segment (start 159.766 54.102) (end 156.972 56.896) (width 1) (layer "B.Cu") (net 3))
 (segment (start 169.672 141.406) (end 171.772 141.406) (width 1) (layer "B.Cu") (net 3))
 (segment (start 232.514 130.556) (end 239.014 130.556) (width 1) (layer "B.Cu") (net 3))
 (segment (start 191.77 42.926) (end 192.786 43.942) (width 1) (layer "B.Cu") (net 3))
 (segment (start 199.208 150.296) (end 232.006 150.296) (width 1) (layer "B.Cu") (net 3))
 (segment (start 244.276 140.644) (end 244.348 140.716) (width 1) (layer "B.Cu") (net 3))
 (segment (start 238.506 94.488) (end 244.348 100.33) (width 1) (layer "B.Cu") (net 3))
 (segment (start 244.094 88.9) (end 244.094 70.612) (width 1) (layer "B.Cu") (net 3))
 (segment (start 159.766 46.99) (end 159.766 54.102) (width 1) (layer "B.Cu") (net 3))
 (segment (start 187.706 46.99) (end 187.706 44.704) (width 1) (layer "B.Cu") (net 3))
 (segment (start 192.786 48.49) (end 202.208 57.912) (width 1) (layer "B.Cu") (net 3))
 (segment (start 192.786 46.99) (end 192.786 48.49) (width 1) (layer "B.Cu") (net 3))
 (segment (start 224.79 57.912) (end 209.55 57.912) (width 1) (layer "B.Cu") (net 3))
 (segment (start 189.484 42.926) (end 191.77 42.926) (width 1) (layer "B.Cu") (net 3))
 (segment (start 187.706 44.704) (end 189.484 42.926) (width 1) (layer "B.Cu") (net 3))
 (segment (start 192.346 150.332) (end 192.382 150.368) (width 1) (layer "B.Cu") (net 3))
 (segment (start 224.536 63.565) (end 224.536 58.166) (width 1) (layer "B.Cu") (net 3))
 (segment (start 244.276 150.296) (end 232.006 150.296) (width 1) (layer "B.Cu") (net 3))
 (segment (start 238.506 140.644) (end 244.276 140.644) (width 1) (layer "B.Cu") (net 3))
 (segment (start 244.348 109.474) (end 244.348 113.03) (width 1) (layer "B.Cu") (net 3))
 (segment (start 243.768 130.738) (end 244.348 131.318) (width 1) (layer "B.Cu") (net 3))
 (segment (start 244.348 140.716) (end 244.348 150.368) (width 1) (layer "B.Cu") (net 3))
 (segment (start 232.26 110.164) (end 238.76 110.164) (width 1) (layer "B.Cu") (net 3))
 (segment (start 238.76 120.324) (end 243.768 120.324) (width 1) (layer "B.Cu") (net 3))
 (segment (start 209.55 57.912) (end 208.788 57.912) (width 1) (layer "B.Cu") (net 3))
 (segment (start 238.76 140.462) (end 238.962 140.26) (width 1) (layer "B.Cu") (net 3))
 (segment (start 238.76 110.164) (end 243.658 110.164) (width 1) (layer "B.Cu") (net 3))
 (segment (start 192.786 43.942) (end 192.786 46.99) (width 1) (layer "B.Cu") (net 3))
 (segment (start 244.348 131.318) (end 244.348 140.716) (width 1) (layer "B.Cu") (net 3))
 (segment (start 238.506 94.488) (end 244.094 88.9) (width 1) (layer "B.Cu") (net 3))
 (segment (start 243.658 110.164) (end 244.348 109.474) (width 1) (layer "B.Cu") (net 3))
 (segment (start 243.768 120.324) (end 244.348 120.904) (width 1) (layer "B.Cu") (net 3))
 (segment (start 243.586 70.104) (end 244.094 70.612) (width 1) (layer "B.Cu") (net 3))
 (segment (start 244.348 120.904) (end 244.348 131.318) (width 1) (layer "B.Cu") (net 3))
 (segment (start 156.972 56.896) (end 156.972 68.834) (width 1) (layer "B.Cu") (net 3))
 (segment (start 232.26 150.114) (end 238.76 150.114) (width 1) (layer "B.Cu") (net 3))
 (segment (start 224.536 58.166) (end 224.79 57.912) (width 1) (layer "B.Cu") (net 3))
 (segment (start 180.698 150.332) (end 187.198 150.332) (width 1) (layer "B.Cu") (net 3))
 (segment (start 154.536 150.042) (end 161.036 150.042) (width 1) (layer "B.Cu") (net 3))
 (segment (start 171.772 141.406) (end 180.698 150.332) (width 1) (layer "B.Cu") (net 3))
 (segment (start 192.382 150.368) (end 198.882 150.368) (width 1) (layer "B.Cu") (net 3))
 (segment (start 244.094 57.912) (end 224.79 57.912) (width 1) (layer "B.Cu") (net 3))
 (segment (start 187.198 150.332) (end 192.346 150.332) (width 1) (layer "B.Cu") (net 3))
 (segment (start 232.462 140.26) (end 238.962 140.26) (width 1) (layer "B.Cu") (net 3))
 (segment (start 244.094 70.612) (end 244.094 57.912) (width 1) (layer "B.Cu") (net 3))
 (segment (start 208.788 57.912) (end 197.866 46.99) (width 1) (layer "B.Cu") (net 3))
 (segment (start 189.992 127.254) (end 189.992 119.888) (width 1) (layer "B.Cu") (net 45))
 (segment (start 190.246 119.634) (end 223.774 119.634) (width 1) (layer "B.Cu") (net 45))
 (segment (start 232.462 135.76) (end 238.962 135.76) (width 1) (layer "B.Cu") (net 45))
 (segment (start 189.992 119.888) (end 190.246 119.634) (width 1) (layer "B.Cu") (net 45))
 (segment (start 223.774 127.072) (end 232.462 135.76) (width 1) (layer "B.Cu") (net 45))
 (segment (start 223.774 119.634) (end 223.774 127.072) (width 1) (layer "B.Cu") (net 45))
 (segment (start 230.466 105.664) (end 232.26 105.664) (width 1) (layer "B.Cu") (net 44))
 (segment (start 230.466 105.664) (end 185.42 105.664) (width 1) (layer "B.Cu") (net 44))
 (segment (start 185.42 105.664) (end 182.372 108.712) (width 1) (layer "B.Cu") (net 44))
 (segment (start 182.372 127.254) (end 182.372 108.712) (width 1) (layer "B.Cu") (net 44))
 (segment (start 238.76 105.664) (end 230.466 105.664) (width 1) (layer "B.Cu") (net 44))
 (segment (start 192.532 127.254) (end 221.234 127.254) (width 1) (layer "B.Cu") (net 50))
 (segment (start 239.014 145.614) (end 232.514 145.614) (width 1) (layer "B.Cu") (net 50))
 (segment (start 221.234 127.254) (end 221.234 134.334) (width 1) (layer "B.Cu") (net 50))
 (segment (start 221.234 134.334) (end 232.514 145.614) (width 1) (layer "B.Cu") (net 50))
 (segment (start 162.052 34.798) (end 162.306 35.052) (width 1) (layer "B.Cu") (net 1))
 (segment (start 127 166.116) (end 126.165 165.281) (width 1) (layer "B.Cu") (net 1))
 (segment (start 162.306 35.052) (end 162.306 46.99) (width 1) (layer "B.Cu") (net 1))
 (segment (start 167.132 127.254) (end 167.132 117.348) (width 1) (layer "B.Cu") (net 1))
 (segment (start 126.165 35.125) (end 126.492 34.798) (width 1) (layer "B.Cu") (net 1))
 (segment (start 126.165 114.808) (end 126.165 83.82) (width 1) (layer "B.Cu") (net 1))
 (segment (start 165.1 114.808) (end 126.165 114.808) (width 1) (layer "B.Cu") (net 1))
 (segment (start 167.132 116.84) (end 165.1 114.808) (width 1) (layer "B.Cu") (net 1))
 (segment (start 167.132 117.348) (end 167.132 116.84) (width 1) (layer "B.Cu") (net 1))
 (segment (start 126.165 83.82) (end 126.165 35.125) (width 1) (layer "B.Cu") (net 1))
 (segment (start 195.326 38.1) (end 192.024 34.798) (width 1) (layer "B.Cu") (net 1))
 (segment (start 195.326 46.99) (end 195.326 38.1) (width 1) (layer "B.Cu") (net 1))
 (segment (start 222.758 83.82) (end 126.165 83.82) (width 1) (layer "B.Cu") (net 1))
 (segment (start 126.492 34.798) (end 162.052 34.798) (width 1) (layer "B.Cu") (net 1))
 (segment (start 233.426 94.488) (end 222.758 83.82) (width 1) (layer "B.Cu") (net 1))
 (segment (start 192.024 34.798) (end 162.052 34.798) (width 1) (layer "B.Cu") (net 1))
 (segment (start 224.568 118.11) (end 232.514 126.056) (width 1) (layer "B.Cu") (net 48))
 (segment (start 187.452 127.254) (end 187.452 118.11) (width 1) (layer "B.Cu") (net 48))
 (segment (start 187.96 118.11) (end 224.568 118.11) (width 1) (layer "B.Cu") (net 48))
 (segment (start 232.514 126.056) (end 239.014 126.056) (width 1) (layer "B.Cu") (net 48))
 (segment (start 187.452 118.11) (end 187.706 117.856) (width 1) (layer "B.Cu") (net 48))
 (segment (start 187.706 117.856) (end 187.96 118.11) (width 1) (layer "B.Cu") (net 48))
 (segment (start 193.222 94.306) (end 220.218 94.306) (width 1) (layer "B.Cu") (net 2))
 (segment (start 179.832 127.254) (end 179.832 107.696) (width 1) (layer "B.Cu") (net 2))
 (segment (start 179.832 107.696) (end 193.222 94.306) (width 1) (layer "B.Cu") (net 2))
 (segment (start 224.464 98.552) (end 235.712 98.552) (width 1) (layer "B.Cu") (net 2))
 (segment (start 235.712 98.552) (end 235.966 98.298) (width 1) (layer "B.Cu") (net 2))
 (segment (start 220.218 94.306) (end 224.464 98.552) (width 1) (layer "B.Cu") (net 2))
 (segment (start 235.966 98.298) (end 235.966 94.488) (width 1) (layer "B.Cu") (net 2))
 (segment (start 154.536 132.946) (end 154.536 145.542) (width 1) (layer "B.Cu") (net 47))
 (segment (start 167.386 130.048) (end 167.386 132.08) (width 1) (layer "B.Cu") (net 47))
 (segment (start 154.432 132.842) (end 154.536 132.946) (width 1) (layer "B.Cu") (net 47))
 (segment (start 167.386 132.08) (end 166.624 132.842) (width 1) (layer "B.Cu") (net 47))
 (segment (start 166.624 132.842) (end 154.432 132.842) (width 1) (layer "B.Cu") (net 47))
 (segment (start 167.132 129.794) (end 167.386 130.048) (width 1) (layer "B.Cu") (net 47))
 (segment (start 161.036 145.542) (end 154.536 145.542) (width 1) (layer "B.Cu") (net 47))
 (segment (start 180.698 145.832) (end 187.198 145.832) (width 1) (layer "B.Cu") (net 49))
 (segment (start 187.198 132.588) (end 187.198 145.832) (width 1) (layer "B.Cu") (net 49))
 (segment (start 189.992 129.794) (end 187.198 132.588) (width 1) (layer "B.Cu") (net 49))
 (segment (start 219.319208 63.939) (end 223.263208 67.883) (width 1) (layer "B.Cu") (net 30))
 (segment (start 182.372 68.834) (end 182.372 63.939) (width 1) (layer "B.Cu") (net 30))
 (segment (start 223.263208 67.883) (end 224.536 67.883) (width 1) (layer "B.Cu") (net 30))
 (segment (start 182.372 63.939) (end 219.319208 63.939) (width 1) (layer "B.Cu") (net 30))
 (segment (start 169.926 68.58) (end 169.672 68.834) (width 1) (layer "B.Cu") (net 21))
 (segment (start 169.926 46.99) (end 169.926 68.58) (width 1) (layer "B.Cu") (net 21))
 (segment (start 172.466 68.58) (end 172.212 68.834) (width 1) (layer "B.Cu") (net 22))
 (segment (start 172.466 46.99) (end 172.466 68.58) (width 1) (layer "B.Cu") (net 22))
 (segment (start 164.846 68.58) (end 164.592 68.834) (width 1) (layer "B.Cu") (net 17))
 (segment (start 164.846 46.99) (end 164.846 68.58) (width 1) (layer "B.Cu") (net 17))
 (segment (start 183.134 57.912) (end 174.752 57.912) (width 1) (layer "B.Cu") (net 24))
 (segment (start 185.166 46.99) (end 185.166 55.88) (width 1) (layer "B.Cu") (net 24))
 (segment (start 185.166 55.88) (end 183.134 57.912) (width 1) (layer "B.Cu") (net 24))
 (segment (start 174.752 57.912) (end 174.752 68.834) (width 1) (layer "B.Cu") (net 24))
 (segment (start 167.386 68.58) (end 167.132 68.834) (width 1) (layer "B.Cu") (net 19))
 (segment (start 167.386 46.99) (end 167.386 68.58) (width 1) (layer "B.Cu") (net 19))
 (segment (start 185.42 60.452) (end 177.546 60.452) (width 1) (layer "B.Cu") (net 26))
 (segment (start 190.246 46.99) (end 190.246 55.626) (width 1) (layer "B.Cu") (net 26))
 (segment (start 177.292 60.198) (end 177.292 68.834) (width 1) (layer "B.Cu") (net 26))
 (segment (start 190.246 55.626) (end 185.42 60.452) (width 1) (layer "B.Cu") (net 26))
 (segment (start 177.546 60.452) (end 177.292 60.198) (width 1) (layer "B.Cu") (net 26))
 (segment (start 187.452 66.294) (end 188.214 65.532) (width 1) (layer "B.Cu") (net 34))
 (segment (start 211.457792 65.532) (end 215.967792 70.042) (width 1) (layer "B.Cu") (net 34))
 (segment (start 215.967792 70.042) (end 224.536 70.042) (width 1) (layer "B.Cu") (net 34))
 (segment (start 187.452 68.834) (end 187.452 66.294) (width 1) (layer "B.Cu") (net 34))
 (segment (start 188.214 65.532) (end 211.457792 65.532) (width 1) (layer "B.Cu") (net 34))
 (segment (start 224.536 65.724) (end 224.536 66.04) (width 1) (layer "B.Cu") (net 28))
 (segment (start 224.282 66.04) (end 220.268 62.026) (width 1) (layer "B.Cu") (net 28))
 (segment (start 224.536 66.04) (end 224.282 66.04) (width 1) (layer "B.Cu") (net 28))
 (segment (start 179.832 62.992) (end 179.832 68.834) (width 1) (layer "B.Cu") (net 28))
 (segment (start 180.798 62.026) (end 179.832 62.992) (width 1) (layer "B.Cu") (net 28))
 (segment (start 220.268 62.026) (end 180.798 62.026) (width 1) (layer "B.Cu") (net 28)))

